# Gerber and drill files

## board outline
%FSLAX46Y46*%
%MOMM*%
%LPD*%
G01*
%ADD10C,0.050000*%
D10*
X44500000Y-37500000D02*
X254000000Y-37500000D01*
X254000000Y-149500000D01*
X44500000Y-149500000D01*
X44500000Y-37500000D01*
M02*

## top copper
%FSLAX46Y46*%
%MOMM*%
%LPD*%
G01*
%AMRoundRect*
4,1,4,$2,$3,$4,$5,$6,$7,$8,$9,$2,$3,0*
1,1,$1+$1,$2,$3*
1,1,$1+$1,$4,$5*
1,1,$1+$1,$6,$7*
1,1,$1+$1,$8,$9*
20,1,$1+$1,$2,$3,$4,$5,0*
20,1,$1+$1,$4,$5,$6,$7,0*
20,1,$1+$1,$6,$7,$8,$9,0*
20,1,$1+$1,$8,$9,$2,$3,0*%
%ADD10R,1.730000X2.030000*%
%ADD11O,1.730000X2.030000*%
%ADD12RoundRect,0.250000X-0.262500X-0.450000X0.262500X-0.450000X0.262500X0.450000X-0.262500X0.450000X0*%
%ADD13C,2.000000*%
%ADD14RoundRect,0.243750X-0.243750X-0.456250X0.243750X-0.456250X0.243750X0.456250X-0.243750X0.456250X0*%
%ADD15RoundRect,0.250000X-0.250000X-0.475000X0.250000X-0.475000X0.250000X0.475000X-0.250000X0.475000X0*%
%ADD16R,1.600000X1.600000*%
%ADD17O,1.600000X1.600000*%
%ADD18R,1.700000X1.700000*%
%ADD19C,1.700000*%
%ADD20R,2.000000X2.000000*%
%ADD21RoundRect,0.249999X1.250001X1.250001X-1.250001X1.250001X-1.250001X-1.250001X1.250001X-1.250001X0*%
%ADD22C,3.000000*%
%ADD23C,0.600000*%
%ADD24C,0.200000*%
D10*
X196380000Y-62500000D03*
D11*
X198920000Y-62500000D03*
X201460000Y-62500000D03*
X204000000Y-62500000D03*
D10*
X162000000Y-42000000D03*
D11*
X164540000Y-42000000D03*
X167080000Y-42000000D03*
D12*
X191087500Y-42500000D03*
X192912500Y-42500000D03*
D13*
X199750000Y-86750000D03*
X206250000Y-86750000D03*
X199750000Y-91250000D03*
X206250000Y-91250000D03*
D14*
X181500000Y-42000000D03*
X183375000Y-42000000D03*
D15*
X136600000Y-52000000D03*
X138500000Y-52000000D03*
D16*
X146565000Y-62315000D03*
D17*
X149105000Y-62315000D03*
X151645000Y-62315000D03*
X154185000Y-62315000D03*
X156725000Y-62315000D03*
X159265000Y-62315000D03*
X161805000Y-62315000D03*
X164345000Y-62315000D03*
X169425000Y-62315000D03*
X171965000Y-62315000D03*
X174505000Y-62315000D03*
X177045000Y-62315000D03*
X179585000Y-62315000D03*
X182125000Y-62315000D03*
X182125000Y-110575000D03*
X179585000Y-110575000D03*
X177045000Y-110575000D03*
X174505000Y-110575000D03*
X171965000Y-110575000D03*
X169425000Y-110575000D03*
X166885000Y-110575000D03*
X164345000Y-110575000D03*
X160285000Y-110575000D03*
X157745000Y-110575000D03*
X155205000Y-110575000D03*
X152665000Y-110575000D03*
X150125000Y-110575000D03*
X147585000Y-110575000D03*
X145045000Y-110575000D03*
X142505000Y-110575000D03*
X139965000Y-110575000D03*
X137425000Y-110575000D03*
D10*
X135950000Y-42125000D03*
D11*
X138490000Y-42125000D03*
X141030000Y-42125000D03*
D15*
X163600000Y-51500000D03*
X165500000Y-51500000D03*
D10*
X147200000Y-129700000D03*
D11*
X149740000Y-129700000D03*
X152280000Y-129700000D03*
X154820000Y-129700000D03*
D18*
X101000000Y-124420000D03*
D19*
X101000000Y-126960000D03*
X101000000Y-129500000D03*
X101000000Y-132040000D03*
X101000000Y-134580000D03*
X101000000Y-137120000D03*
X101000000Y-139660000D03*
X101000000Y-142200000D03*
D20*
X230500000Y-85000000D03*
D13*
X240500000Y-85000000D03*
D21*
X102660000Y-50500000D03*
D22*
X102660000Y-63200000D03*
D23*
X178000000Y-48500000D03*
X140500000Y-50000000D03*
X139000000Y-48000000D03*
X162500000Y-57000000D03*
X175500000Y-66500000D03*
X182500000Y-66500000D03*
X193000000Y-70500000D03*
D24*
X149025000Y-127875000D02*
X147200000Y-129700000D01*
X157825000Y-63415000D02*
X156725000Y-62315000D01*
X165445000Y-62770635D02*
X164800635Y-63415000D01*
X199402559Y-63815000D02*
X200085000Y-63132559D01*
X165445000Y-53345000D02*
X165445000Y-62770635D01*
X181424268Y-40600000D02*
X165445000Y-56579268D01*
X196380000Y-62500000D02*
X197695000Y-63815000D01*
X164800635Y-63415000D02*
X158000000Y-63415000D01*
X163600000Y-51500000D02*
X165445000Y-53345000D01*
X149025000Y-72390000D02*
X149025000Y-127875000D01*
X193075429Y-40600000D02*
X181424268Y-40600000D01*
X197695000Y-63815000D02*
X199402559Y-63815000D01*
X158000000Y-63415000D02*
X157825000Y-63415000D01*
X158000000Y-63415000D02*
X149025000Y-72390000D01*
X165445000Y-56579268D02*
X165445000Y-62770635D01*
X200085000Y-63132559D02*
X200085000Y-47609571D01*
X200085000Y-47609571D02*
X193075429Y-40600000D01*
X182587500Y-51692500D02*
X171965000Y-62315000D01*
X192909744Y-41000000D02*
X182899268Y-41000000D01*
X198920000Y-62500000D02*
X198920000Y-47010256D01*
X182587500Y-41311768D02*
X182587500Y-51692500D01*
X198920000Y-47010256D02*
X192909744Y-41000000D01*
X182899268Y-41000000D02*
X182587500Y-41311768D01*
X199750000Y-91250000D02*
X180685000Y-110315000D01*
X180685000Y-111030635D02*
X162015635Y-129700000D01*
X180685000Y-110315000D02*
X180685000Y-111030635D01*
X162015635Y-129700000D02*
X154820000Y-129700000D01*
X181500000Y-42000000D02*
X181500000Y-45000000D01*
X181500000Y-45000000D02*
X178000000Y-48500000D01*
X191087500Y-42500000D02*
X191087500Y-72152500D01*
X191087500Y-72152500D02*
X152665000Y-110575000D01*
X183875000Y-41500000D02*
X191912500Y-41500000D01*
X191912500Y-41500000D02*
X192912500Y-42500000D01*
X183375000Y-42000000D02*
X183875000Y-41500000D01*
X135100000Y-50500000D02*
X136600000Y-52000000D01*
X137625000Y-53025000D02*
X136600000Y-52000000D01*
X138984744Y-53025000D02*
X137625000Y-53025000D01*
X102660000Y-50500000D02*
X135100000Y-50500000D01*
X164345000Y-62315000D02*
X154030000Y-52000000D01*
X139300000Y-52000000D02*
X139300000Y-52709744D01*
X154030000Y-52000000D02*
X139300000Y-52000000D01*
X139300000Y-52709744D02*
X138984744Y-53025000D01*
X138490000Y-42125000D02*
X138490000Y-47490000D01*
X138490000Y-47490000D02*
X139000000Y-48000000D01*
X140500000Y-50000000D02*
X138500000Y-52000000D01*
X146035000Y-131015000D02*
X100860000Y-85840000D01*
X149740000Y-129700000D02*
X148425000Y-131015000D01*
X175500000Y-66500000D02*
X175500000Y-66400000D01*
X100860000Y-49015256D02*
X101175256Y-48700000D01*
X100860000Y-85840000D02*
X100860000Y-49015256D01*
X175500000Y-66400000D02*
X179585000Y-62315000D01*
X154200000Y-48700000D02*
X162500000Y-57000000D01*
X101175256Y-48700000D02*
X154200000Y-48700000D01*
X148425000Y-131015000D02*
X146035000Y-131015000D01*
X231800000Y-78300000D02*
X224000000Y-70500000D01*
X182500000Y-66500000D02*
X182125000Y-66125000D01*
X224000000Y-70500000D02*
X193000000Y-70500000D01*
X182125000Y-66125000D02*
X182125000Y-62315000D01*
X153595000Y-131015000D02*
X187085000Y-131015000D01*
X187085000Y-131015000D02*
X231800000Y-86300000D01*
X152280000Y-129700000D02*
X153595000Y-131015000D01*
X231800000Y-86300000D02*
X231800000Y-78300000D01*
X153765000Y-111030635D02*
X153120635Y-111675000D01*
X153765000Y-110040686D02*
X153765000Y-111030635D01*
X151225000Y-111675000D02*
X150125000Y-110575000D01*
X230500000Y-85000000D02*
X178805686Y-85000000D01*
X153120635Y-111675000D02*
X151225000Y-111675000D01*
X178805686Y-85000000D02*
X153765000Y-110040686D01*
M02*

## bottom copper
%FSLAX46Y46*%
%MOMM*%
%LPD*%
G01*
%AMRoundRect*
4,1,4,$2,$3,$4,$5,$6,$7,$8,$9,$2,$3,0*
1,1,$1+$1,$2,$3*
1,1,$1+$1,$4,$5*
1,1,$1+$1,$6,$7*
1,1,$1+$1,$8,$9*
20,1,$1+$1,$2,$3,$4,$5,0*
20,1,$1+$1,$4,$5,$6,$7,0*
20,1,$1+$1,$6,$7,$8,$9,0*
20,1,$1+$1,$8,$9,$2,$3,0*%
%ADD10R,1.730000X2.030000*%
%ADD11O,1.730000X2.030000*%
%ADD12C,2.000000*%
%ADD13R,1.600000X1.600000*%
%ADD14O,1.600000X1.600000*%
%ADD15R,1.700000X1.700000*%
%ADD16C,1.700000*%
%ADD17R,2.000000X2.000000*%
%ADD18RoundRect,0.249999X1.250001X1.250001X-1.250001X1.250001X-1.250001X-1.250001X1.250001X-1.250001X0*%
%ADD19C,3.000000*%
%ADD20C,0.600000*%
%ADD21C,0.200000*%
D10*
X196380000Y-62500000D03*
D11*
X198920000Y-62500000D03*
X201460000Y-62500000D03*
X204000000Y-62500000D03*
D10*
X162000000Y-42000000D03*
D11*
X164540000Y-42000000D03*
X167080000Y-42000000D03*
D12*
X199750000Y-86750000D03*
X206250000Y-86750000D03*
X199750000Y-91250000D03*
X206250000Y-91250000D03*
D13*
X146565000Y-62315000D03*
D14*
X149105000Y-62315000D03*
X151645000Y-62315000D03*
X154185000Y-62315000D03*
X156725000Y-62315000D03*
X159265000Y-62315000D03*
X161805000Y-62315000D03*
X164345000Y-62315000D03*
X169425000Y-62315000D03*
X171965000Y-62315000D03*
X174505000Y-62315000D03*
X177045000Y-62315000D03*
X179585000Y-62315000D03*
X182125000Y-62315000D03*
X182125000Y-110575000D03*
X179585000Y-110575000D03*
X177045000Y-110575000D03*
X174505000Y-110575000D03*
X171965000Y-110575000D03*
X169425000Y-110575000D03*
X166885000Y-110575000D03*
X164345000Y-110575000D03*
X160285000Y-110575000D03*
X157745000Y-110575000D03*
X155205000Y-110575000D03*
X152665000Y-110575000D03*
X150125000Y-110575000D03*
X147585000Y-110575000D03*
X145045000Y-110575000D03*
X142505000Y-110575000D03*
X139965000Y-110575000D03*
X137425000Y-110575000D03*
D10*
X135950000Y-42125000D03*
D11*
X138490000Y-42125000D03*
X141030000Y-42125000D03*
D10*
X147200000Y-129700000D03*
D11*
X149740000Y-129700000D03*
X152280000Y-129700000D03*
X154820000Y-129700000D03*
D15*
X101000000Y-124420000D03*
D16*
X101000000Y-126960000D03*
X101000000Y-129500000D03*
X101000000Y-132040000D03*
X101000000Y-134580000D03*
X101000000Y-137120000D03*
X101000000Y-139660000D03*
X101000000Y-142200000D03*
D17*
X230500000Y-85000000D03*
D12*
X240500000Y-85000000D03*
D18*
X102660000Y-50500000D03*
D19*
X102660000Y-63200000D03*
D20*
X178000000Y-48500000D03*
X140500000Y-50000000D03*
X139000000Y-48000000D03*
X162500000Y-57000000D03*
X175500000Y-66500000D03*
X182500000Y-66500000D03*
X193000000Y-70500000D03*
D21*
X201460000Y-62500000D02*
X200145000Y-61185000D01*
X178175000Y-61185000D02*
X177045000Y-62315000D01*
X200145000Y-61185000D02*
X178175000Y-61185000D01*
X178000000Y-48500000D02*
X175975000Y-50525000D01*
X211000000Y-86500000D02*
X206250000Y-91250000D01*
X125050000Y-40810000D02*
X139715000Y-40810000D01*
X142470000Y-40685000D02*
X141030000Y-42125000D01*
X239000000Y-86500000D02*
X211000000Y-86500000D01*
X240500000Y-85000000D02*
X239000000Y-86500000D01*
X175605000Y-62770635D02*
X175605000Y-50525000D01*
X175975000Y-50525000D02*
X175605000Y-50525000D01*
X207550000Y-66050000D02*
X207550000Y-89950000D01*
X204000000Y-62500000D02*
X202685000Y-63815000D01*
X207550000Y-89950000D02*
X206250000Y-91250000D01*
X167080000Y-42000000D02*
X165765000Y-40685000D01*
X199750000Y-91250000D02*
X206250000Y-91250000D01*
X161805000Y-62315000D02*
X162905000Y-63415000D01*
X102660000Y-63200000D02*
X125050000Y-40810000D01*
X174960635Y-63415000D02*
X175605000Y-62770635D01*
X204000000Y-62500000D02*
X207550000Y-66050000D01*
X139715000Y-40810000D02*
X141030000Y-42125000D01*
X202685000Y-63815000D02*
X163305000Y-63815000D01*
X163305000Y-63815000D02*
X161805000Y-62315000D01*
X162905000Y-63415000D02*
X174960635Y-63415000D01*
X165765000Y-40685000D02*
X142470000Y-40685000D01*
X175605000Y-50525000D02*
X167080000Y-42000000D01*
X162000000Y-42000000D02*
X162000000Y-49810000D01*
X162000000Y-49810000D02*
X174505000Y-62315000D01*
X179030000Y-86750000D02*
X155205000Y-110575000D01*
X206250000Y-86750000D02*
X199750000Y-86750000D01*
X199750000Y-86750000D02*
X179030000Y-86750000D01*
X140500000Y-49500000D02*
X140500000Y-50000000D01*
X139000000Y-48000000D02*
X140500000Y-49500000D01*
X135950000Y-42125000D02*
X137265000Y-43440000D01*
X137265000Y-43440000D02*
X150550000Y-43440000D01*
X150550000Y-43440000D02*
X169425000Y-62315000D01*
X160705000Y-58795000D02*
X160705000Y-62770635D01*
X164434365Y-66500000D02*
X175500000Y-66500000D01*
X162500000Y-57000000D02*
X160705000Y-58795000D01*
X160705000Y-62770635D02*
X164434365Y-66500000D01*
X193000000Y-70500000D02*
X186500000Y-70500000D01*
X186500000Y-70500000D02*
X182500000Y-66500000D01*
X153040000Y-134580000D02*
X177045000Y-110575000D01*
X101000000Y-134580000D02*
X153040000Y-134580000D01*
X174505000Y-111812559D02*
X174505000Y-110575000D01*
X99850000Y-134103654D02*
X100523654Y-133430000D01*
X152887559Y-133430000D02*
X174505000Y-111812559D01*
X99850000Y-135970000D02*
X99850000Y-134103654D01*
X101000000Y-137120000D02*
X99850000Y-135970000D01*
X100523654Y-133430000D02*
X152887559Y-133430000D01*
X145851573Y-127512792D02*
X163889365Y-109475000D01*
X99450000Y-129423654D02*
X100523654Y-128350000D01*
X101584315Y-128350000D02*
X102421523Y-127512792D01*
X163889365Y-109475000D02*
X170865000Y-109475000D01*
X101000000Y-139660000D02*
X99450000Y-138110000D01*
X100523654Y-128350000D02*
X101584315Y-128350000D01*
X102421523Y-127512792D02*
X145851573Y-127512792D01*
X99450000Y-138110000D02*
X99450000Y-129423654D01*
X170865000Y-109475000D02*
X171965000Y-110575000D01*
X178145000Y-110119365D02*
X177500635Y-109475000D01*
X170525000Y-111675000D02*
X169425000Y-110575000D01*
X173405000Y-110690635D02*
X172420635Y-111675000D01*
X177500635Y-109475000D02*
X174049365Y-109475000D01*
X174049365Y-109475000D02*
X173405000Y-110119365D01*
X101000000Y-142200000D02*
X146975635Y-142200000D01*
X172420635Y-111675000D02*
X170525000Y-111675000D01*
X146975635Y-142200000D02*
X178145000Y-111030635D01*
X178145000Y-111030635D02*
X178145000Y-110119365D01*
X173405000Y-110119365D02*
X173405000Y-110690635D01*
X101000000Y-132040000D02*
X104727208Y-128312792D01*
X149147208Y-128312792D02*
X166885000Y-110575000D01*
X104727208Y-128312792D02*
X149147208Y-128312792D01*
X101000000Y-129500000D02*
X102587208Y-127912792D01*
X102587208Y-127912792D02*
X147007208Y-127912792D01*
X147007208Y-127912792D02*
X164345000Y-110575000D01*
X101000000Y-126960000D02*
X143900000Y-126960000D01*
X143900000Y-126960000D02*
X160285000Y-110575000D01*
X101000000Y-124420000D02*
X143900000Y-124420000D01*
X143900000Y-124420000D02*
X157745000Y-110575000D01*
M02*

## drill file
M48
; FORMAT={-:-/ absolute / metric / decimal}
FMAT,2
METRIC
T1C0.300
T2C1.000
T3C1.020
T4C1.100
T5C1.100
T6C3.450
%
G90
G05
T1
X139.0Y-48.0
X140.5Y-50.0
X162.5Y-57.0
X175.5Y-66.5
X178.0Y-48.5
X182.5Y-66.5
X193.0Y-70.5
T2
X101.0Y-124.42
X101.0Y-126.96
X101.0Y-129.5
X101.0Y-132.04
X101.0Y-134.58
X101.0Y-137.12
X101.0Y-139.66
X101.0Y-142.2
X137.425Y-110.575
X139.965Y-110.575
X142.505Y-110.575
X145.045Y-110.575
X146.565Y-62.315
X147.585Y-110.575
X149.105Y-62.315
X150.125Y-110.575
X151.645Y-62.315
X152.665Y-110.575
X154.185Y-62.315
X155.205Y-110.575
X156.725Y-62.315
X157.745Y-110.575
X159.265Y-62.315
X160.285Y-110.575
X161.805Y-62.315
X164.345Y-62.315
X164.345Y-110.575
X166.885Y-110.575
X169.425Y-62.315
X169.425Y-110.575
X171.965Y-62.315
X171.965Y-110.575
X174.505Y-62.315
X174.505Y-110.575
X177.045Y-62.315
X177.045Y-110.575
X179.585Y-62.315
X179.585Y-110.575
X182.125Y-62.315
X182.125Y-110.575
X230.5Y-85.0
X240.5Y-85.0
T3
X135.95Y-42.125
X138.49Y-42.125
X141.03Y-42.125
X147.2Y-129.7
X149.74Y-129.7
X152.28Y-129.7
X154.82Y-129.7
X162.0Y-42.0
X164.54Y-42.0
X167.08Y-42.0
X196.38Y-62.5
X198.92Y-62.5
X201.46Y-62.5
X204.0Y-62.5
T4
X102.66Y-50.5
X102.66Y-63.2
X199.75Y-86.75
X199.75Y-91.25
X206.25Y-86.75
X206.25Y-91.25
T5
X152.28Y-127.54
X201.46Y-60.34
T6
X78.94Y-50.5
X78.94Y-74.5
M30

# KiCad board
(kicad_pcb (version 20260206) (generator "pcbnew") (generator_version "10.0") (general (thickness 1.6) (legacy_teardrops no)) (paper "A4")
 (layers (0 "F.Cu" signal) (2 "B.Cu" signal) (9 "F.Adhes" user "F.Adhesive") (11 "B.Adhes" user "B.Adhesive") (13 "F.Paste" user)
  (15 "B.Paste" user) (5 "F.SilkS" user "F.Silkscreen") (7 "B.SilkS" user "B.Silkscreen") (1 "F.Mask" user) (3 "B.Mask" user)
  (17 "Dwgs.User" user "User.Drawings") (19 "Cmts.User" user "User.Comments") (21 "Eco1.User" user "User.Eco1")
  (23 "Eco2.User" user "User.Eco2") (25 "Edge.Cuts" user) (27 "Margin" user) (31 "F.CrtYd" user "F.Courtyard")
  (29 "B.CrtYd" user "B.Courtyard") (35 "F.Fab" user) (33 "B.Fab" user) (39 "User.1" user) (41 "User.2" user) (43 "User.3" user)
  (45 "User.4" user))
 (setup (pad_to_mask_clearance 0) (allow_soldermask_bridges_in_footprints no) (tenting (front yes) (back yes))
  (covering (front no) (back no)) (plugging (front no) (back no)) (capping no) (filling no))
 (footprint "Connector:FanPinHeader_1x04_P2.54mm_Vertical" (layer "F.Cu") (at 196.38 62.5)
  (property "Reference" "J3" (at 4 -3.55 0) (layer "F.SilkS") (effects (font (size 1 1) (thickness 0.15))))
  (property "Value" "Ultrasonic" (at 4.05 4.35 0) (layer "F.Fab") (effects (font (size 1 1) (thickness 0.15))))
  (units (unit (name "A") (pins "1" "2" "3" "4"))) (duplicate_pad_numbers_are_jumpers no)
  (pad "" np_thru_hole circle (at 5.08 -2.16 90) (size 1.1 1.1) (drill 1.1) (layers "*.Cu" "*.Mask"))
  (pad "1" thru_hole rect (at 0 0 90) (size 2.03 1.73) (drill 1.02) (layers "*.Cu" "*.Mask") (remove_unused_layers no) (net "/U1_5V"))
  (pad "2" thru_hole oval (at 2.54 0 90) (size 2.03 1.73) (drill 1.02) (layers "*.Cu" "*.Mask") (remove_unused_layers no)
   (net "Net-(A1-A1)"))
  (pad "3" thru_hole oval (at 5.08 0 90) (size 2.03 1.73) (drill 1.02) (layers "*.Cu" "*.Mask") (remove_unused_layers no)
   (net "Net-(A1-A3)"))
  (pad "4" thru_hole oval (at 7.62 0 90) (size 2.03 1.73) (drill 1.02) (layers "*.Cu" "*.Mask") (remove_unused_layers no) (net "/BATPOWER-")))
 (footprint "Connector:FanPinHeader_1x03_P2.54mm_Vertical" (layer "F.Cu") (at 162 42)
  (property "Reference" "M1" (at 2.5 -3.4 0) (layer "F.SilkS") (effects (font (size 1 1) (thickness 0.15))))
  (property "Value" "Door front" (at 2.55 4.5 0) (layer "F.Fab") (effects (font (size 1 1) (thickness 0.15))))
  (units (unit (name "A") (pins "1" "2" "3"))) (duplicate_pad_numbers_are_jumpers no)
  (pad "1" thru_hole rect (at 0 0 90) (size 2.03 1.73) (drill 1.02) (layers "*.Cu" "*.Mask") (remove_unused_layers no) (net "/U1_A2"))
  (pad "2" thru_hole oval (at 2.54 0 90) (size 2.03 1.73) (drill 1.02) (layers "*.Cu" "*.Mask") (remove_unused_layers no) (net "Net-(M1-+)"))
  (pad "3" thru_hole oval (at 5.08 0 90) (size 2.03 1.73) (drill 1.02) (layers "*.Cu" "*.Mask") (remove_unused_layers no) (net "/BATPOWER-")))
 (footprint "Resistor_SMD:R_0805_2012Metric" (layer "F.Cu") (at 192 42.5)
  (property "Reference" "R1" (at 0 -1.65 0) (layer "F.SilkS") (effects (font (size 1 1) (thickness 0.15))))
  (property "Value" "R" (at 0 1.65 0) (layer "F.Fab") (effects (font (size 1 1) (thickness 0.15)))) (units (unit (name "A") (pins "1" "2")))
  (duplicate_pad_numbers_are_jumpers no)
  (pad "1" smd roundrect (at -0.9125 0) (size 1.025 1.4) (layers "F.Cu" "F.Mask" "F.Paste") (roundrect_rratio 0.243902) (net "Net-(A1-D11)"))
  (pad "2" smd roundrect (at 0.9125 0) (size 1.025 1.4) (layers "F.Cu" "F.Mask" "F.Paste") (roundrect_rratio 0.243902) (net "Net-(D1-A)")))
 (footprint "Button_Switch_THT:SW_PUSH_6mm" (layer "F.Cu") (at 199.75 86.75)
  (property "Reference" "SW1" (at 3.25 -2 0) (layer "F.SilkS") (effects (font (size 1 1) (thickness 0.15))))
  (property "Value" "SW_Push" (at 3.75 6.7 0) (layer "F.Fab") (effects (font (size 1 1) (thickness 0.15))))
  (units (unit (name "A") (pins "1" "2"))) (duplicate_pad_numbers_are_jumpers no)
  (pad "1" thru_hole circle (at 0 0 90) (size 2 2) (drill 1.1) (layers "*.Cu" "*.Mask") (remove_unused_layers no) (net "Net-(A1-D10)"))
  (pad "1" thru_hole circle (at 6.5 0 90) (size 2 2) (drill 1.1) (layers "*.Cu" "*.Mask") (remove_unused_layers no) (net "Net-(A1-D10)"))
  (pad "2" thru_hole circle (at 0 4.5 90) (size 2 2) (drill 1.1) (layers "*.Cu" "*.Mask") (remove_unused_layers no) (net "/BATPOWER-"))
  (pad "2" thru_hole circle (at 6.5 4.5 90) (size 2 2) (drill 1.1) (layers "*.Cu" "*.Mask") (remove_unused_layers no) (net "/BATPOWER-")))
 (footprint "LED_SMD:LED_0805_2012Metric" (layer "F.Cu") (at 182.4375 42)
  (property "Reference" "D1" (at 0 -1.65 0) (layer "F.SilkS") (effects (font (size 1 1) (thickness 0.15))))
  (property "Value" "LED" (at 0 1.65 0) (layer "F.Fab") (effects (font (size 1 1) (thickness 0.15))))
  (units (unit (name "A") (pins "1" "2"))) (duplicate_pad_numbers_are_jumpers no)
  (pad "1" smd roundrect (at -0.9375 0) (size 0.975 1.4) (layers "F.Cu" "F.Mask" "F.Paste") (roundrect_rratio 0.25) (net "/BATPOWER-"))
  (pad "2" smd roundrect (at 0.9375 0) (size 0.975 1.4) (layers "F.Cu" "F.Mask" "F.Paste") (roundrect_rratio 0.25) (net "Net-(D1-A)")))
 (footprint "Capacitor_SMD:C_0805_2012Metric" (layer "F.Cu") (at 137.55 52)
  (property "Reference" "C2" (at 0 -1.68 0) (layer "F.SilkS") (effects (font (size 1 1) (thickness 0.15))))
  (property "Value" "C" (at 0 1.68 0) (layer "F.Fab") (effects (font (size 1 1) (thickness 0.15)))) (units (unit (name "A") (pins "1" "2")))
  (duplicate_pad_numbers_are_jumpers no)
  (pad "1" smd roundrect (at -0.95 0) (size 1 1.45) (layers "F.Cu" "F.Mask" "F.Paste") (roundrect_rratio 0.25) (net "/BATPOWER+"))
  (pad "2" smd roundrect (at 0.95 0) (size 1 1.45) (layers "F.Cu" "F.Mask" "F.Paste") (roundrect_rratio 0.25) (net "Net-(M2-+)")))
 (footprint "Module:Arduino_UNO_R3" (layer "F.Cu") (at 146.565 62.315)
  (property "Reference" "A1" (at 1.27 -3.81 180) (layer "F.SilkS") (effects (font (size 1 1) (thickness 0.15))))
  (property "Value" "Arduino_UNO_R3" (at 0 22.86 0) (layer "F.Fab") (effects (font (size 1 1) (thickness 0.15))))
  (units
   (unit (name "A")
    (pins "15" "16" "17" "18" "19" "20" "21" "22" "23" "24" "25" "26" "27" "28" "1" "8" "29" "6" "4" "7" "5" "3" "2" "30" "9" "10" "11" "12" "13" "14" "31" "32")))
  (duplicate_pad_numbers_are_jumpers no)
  (pad "1" thru_hole rect (at 0 0 90) (size 1.6 1.6) (drill 1) (layers "*.Cu" "*.Mask") (remove_unused_layers no)
   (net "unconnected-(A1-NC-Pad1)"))
  (pad "2" thru_hole oval (at 2.54 0 90) (size 1.6 1.6) (drill 1) (layers "*.Cu" "*.Mask") (remove_unused_layers no)
   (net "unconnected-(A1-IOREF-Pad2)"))
  (pad "3" thru_hole oval (at 5.08 0 90) (size 1.6 1.6) (drill 1) (layers "*.Cu" "*.Mask") (remove_unused_layers no)
   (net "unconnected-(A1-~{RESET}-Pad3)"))
  (pad "4" thru_hole oval (at 7.62 0 90) (size 1.6 1.6) (drill 1) (layers "*.Cu" "*.Mask") (remove_unused_layers no)
   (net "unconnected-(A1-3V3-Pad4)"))
  (pad "5" thru_hole oval (at 10.16 0 90) (size 1.6 1.6) (drill 1) (layers "*.Cu" "*.Mask") (remove_unused_layers no) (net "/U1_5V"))
  (pad "6" thru_hole oval (at 12.7 0 90) (size 1.6 1.6) (drill 1) (layers "*.Cu" "*.Mask") (remove_unused_layers no)
   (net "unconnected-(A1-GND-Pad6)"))
  (pad "7" thru_hole oval (at 15.24 0 90) (size 1.6 1.6) (drill 1) (layers "*.Cu" "*.Mask") (remove_unused_layers no) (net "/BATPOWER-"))
  (pad "8" thru_hole oval (at 17.78 0 90) (size 1.6 1.6) (drill 1) (layers "*.Cu" "*.Mask") (remove_unused_layers no) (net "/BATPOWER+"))
  (pad "9" thru_hole oval (at 22.86 0 90) (size 1.6 1.6) (drill 1) (layers "*.Cu" "*.Mask") (remove_unused_layers no) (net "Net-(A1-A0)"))
  (pad "10" thru_hole oval (at 25.4 0 90) (size 1.6 1.6) (drill 1) (layers "*.Cu" "*.Mask") (remove_unused_layers no) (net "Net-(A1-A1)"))
  (pad "11" thru_hole oval (at 27.94 0 90) (size 1.6 1.6) (drill 1) (layers "*.Cu" "*.Mask") (remove_unused_layers no) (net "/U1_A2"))
  (pad "12" thru_hole oval (at 30.48 0 90) (size 1.6 1.6) (drill 1) (layers "*.Cu" "*.Mask") (remove_unused_layers no) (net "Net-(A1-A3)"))
  (pad "13" thru_hole oval (at 33.02 0 90) (size 1.6 1.6) (drill 1) (layers "*.Cu" "*.Mask") (remove_unused_layers no) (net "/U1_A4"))
  (pad "14" thru_hole oval (at 35.56 0 90) (size 1.6 1.6) (drill 1) (layers "*.Cu" "*.Mask") (remove_unused_layers no) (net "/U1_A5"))
  (pad "15" thru_hole oval (at 35.56 48.26 90) (size 1.6 1.6) (drill 1) (layers "*.Cu" "*.Mask") (remove_unused_layers no)
   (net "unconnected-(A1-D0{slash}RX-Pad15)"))
  (pad "16" thru_hole oval (at 33.02 48.26 90) (size 1.6 1.6) (drill 1) (layers "*.Cu" "*.Mask") (remove_unused_layers no)
   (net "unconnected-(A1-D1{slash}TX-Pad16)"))
  (pad "17" thru_hole oval (at 30.48 48.26 90) (size 1.6 1.6) (drill 1) (layers "*.Cu" "*.Mask") (remove_unused_layers no) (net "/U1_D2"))
  (pad "18" thru_hole oval (at 27.94 48.26 90) (size 1.6 1.6) (drill 1) (layers "*.Cu" "*.Mask") (remove_unused_layers no) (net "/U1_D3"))
  (pad "19" thru_hole oval (at 25.4 48.26 90) (size 1.6 1.6) (drill 1) (layers "*.Cu" "*.Mask") (remove_unused_layers no) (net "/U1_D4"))
  (pad "20" thru_hole oval (at 22.86 48.26 90) (size 1.6 1.6) (drill 1) (layers "*.Cu" "*.Mask") (remove_unused_layers no) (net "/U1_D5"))
  (pad "21" thru_hole oval (at 20.32 48.26 90) (size 1.6 1.6) (drill 1) (layers "*.Cu" "*.Mask") (remove_unused_layers no) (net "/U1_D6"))
  (pad "22" thru_hole oval (at 17.78 48.26 90) (size 1.6 1.6) (drill 1) (layers "*.Cu" "*.Mask") (remove_unused_layers no) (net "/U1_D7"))
  (pad "23" thru_hole oval (at 13.72 48.26 90) (size 1.6 1.6) (drill 1) (layers "*.Cu" "*.Mask") (remove_unused_layers no) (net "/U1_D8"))
  (pad "24" thru_hole oval (at 11.18 48.26 90) (size 1.6 1.6) (drill 1) (layers "*.Cu" "*.Mask") (remove_unused_layers no) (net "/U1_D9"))
  (pad "25" thru_hole oval (at 8.64 48.26 90) (size 1.6 1.6) (drill 1) (layers "*.Cu" "*.Mask") (remove_unused_layers no)
   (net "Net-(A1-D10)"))
  (pad "26" thru_hole oval (at 6.1 48.26 90) (size 1.6 1.6) (drill 1) (layers "*.Cu" "*.Mask") (remove_unused_layers no)
   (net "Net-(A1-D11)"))
  (pad "27" thru_hole oval (at 3.56 48.26 90) (size 1.6 1.6) (drill 1) (layers "*.Cu" "*.Mask") (remove_unused_layers no) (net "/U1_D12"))
  (pad "28" thru_hole oval (at 1.02 48.26 90) (size 1.6 1.6) (drill 1) (layers "*.Cu" "*.Mask") (remove_unused_layers no)
   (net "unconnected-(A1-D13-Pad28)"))
  (pad "29" thru_hole oval (at -1.52 48.26 90) (size 1.6 1.6) (drill 1) (layers "*.Cu" "*.Mask") (remove_unused_layers no)
   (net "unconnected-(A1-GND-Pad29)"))
  (pad "30" thru_hole oval (at -4.06 48.26 90) (size 1.6 1.6) (drill 1) (layers "*.Cu" "*.Mask") (remove_unused_layers no)
   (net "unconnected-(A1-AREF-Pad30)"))
  (pad "31" thru_hole oval (at -6.6 48.26 90) (size 1.6 1.6) (drill 1) (layers "*.Cu" "*.Mask") (remove_unused_layers no)
   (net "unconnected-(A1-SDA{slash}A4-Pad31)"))
  (pad "32" thru_hole oval (at -9.14 48.26 90) (size 1.6 1.6) (drill 1) (layers "*.Cu" "*.Mask") (remove_unused_layers no)
   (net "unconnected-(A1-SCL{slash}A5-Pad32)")))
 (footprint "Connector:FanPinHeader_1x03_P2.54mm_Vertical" (layer "F.Cu") (at 135.95 42.125)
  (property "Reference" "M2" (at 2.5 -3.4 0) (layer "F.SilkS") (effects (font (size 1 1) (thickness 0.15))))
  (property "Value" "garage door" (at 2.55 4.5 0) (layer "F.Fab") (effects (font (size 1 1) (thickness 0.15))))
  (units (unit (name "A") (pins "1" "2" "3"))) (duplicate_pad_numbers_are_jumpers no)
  (pad "1" thru_hole rect (at 0 0 90) (size 2.03 1.73) (drill 1.02) (layers "*.Cu" "*.Mask") (remove_unused_layers no) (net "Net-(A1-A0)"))
  (pad "2" thru_hole oval (at 2.54 0 90) (size 2.03 1.73) (drill 1.02) (layers "*.Cu" "*.Mask") (remove_unused_layers no) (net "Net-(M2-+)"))
  (pad "3" thru_hole oval (at 5.08 0 90) (size 2.03 1.73) (drill 1.02) (layers "*.Cu" "*.Mask") (remove_unused_layers no) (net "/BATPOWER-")))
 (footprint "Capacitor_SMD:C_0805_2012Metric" (layer "F.Cu") (at 164.55 51.5)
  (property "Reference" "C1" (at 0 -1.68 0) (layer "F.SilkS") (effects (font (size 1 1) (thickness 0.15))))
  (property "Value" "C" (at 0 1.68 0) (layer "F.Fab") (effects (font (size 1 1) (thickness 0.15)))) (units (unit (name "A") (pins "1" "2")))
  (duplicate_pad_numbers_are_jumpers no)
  (pad "1" smd roundrect (at -0.95 0) (size 1 1.45) (layers "F.Cu" "F.Mask" "F.Paste") (roundrect_rratio 0.25) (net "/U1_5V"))
  (pad "2" smd roundrect (at 0.95 0) (size 1 1.45) (layers "F.Cu" "F.Mask" "F.Paste") (roundrect_rratio 0.25) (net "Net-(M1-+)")))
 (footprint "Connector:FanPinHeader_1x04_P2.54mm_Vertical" (layer "F.Cu") (at 147.2 129.7)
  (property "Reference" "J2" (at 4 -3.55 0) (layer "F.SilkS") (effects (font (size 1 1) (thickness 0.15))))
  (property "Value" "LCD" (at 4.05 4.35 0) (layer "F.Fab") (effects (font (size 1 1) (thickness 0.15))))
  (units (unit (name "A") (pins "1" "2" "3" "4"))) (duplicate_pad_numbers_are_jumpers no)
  (pad "" np_thru_hole circle (at 5.08 -2.16 90) (size 1.1 1.1) (drill 1.1) (layers "*.Cu" "*.Mask"))
  (pad "1" thru_hole rect (at 0 0 90) (size 2.03 1.73) (drill 1.02) (layers "*.Cu" "*.Mask") (remove_unused_layers no) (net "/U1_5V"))
  (pad "2" thru_hole oval (at 2.54 0 90) (size 2.03 1.73) (drill 1.02) (layers "*.Cu" "*.Mask") (remove_unused_layers no) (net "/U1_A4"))
  (pad "3" thru_hole oval (at 5.08 0 90) (size 2.03 1.73) (drill 1.02) (layers "*.Cu" "*.Mask") (remove_unused_layers no) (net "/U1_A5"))
  (pad "4" thru_hole oval (at 7.62 0 90) (size 2.03 1.73) (drill 1.02) (layers "*.Cu" "*.Mask") (remove_unused_layers no) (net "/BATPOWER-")))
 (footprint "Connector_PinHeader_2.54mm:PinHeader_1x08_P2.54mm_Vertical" (layer "F.Cu") (at 101 124.42)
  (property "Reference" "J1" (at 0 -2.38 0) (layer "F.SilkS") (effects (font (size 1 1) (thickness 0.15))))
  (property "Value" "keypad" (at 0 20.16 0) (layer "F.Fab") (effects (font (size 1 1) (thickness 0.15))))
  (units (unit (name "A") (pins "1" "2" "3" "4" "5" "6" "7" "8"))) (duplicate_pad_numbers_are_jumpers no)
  (pad "1" thru_hole rect (at 0 0) (size 1.7 1.7) (drill 1) (layers "*.Cu" "*.Mask") (remove_unused_layers no) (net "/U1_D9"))
  (pad "2" thru_hole circle (at 0 2.54) (size 1.7 1.7) (drill 1) (layers "*.Cu" "*.Mask") (remove_unused_layers no) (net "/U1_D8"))
  (pad "3" thru_hole circle (at 0 5.08) (size 1.7 1.7) (drill 1) (layers "*.Cu" "*.Mask") (remove_unused_layers no) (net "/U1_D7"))
  (pad "4" thru_hole circle (at 0 7.62) (size 1.7 1.7) (drill 1) (layers "*.Cu" "*.Mask") (remove_unused_layers no) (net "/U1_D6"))
  (pad "5" thru_hole circle (at 0 10.16) (size 1.7 1.7) (drill 1) (layers "*.Cu" "*.Mask") (remove_unused_layers no) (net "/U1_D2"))
  (pad "6" thru_hole circle (at 0 12.7) (size 1.7 1.7) (drill 1) (layers "*.Cu" "*.Mask") (remove_unused_layers no) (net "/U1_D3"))
  (pad "7" thru_hole circle (at 0 15.24) (size 1.7 1.7) (drill 1) (layers "*.Cu" "*.Mask") (remove_unused_layers no) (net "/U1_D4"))
  (pad "8" thru_hole circle (at 0 17.78) (size 1.7 1.7) (drill 1) (layers "*.Cu" "*.Mask") (remove_unused_layers no) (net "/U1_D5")))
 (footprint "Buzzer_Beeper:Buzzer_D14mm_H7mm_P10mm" (layer "F.Cu") (at 230.5 85)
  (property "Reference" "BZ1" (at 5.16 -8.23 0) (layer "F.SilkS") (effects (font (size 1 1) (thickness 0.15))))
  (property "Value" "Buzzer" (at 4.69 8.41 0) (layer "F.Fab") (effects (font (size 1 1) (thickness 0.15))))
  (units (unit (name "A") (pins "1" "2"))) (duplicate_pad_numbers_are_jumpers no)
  (pad "1" thru_hole rect (at 0 0) (size 2 2) (drill 1) (layers "*.Cu" "*.Mask") (remove_unused_layers no) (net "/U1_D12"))
  (pad "2" thru_hole circle (at 10 0) (size 2 2) (drill 1) (layers "*.Cu" "*.Mask") (remove_unused_layers no) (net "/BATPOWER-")))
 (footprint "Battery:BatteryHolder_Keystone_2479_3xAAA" (layer "B.Cu") (at 102.66 50.5 180)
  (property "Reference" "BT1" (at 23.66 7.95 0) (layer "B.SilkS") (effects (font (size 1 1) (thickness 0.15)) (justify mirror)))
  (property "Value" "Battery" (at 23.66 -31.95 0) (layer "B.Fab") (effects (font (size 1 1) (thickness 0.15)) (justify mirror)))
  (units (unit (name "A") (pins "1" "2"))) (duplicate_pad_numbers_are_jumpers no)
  (pad "" np_thru_hole circle (at 23.72 -24 180) (size 3.45 3.45) (drill 3.45) (layers "*.Cu" "*.Mask"))
  (pad "" np_thru_hole circle (at 23.72 0 180) (size 3.45 3.45) (drill 3.45) (layers "*.Cu" "*.Mask"))
  (pad "1" thru_hole roundrect (at 0 0 180) (size 3 3) (drill 1.1) (layers "*.Cu" "*.Mask") (remove_unused_layers no)
   (roundrect_rratio 0.083333) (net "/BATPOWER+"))
  (pad "2" thru_hole circle (at 0 -12.7 180) (size 3 3) (drill 1.1) (layers "*.Cu" "*.Mask") (remove_unused_layers no) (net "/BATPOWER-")))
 (gr_rect (start 44.5 37.5) (end 254 149.5) (stroke (width 0.05) (type default)) (fill no) (layer "Edge.Cuts"))
 (segment (start 149.025 127.875) (end 147.2 129.7) (width 0.2) (layer "F.Cu") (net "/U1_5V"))
 (segment (start 157.825 63.415) (end 156.725 62.315) (width 0.2) (layer "F.Cu") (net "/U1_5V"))
 (segment (start 165.445 62.770635) (end 164.800635 63.415) (width 0.2) (layer "F.Cu") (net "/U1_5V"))
 (segment (start 199.402559 63.815) (end 200.085 63.132559) (width 0.2) (layer "F.Cu") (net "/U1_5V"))
 (segment (start 165.445 53.345) (end 165.445 62.770635) (width 0.2) (layer "F.Cu") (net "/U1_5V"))
 (segment (start 181.424268 40.6) (end 165.445 56.579268) (width 0.2) (layer "F.Cu") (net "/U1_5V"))
 (segment (start 196.38 62.5) (end 197.695 63.815) (width 0.2) (layer "F.Cu") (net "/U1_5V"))
 (segment (start 164.800635 63.415) (end 158 63.415) (width 0.2) (layer "F.Cu") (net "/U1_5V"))
 (segment (start 163.6 51.5) (end 165.445 53.345) (width 0.2) (layer "F.Cu") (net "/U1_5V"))
 (segment (start 149.025 72.39) (end 149.025 127.875) (width 0.2) (layer "F.Cu") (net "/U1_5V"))
 (segment (start 193.075429 40.6) (end 181.424268 40.6) (width 0.2) (layer "F.Cu") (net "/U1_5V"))
 (segment (start 197.695 63.815) (end 199.402559 63.815) (width 0.2) (layer "F.Cu") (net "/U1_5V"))
 (segment (start 158 63.415) (end 157.825 63.415) (width 0.2) (layer "F.Cu") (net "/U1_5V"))
 (segment (start 158 63.415) (end 149.025 72.39) (width 0.2) (layer "F.Cu") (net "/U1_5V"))
 (segment (start 165.445 56.579268) (end 165.445 62.770635) (width 0.2) (layer "F.Cu") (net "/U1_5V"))
 (segment (start 200.085 63.132559) (end 200.085 47.609571) (width 0.2) (layer "F.Cu") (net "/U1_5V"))
 (segment (start 200.085 47.609571) (end 193.075429 40.6) (width 0.2) (layer "F.Cu") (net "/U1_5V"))
 (segment (start 182.5875 51.6925) (end 171.965 62.315) (width 0.2) (layer "F.Cu") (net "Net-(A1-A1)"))
 (segment (start 192.909744 41) (end 182.899268 41) (width 0.2) (layer "F.Cu") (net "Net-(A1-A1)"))
 (segment (start 198.92 62.5) (end 198.92 47.010256) (width 0.2) (layer "F.Cu") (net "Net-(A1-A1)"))
 (segment (start 182.5875 41.311768) (end 182.5875 51.6925) (width 0.2) (layer "F.Cu") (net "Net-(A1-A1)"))
 (segment (start 198.92 47.010256) (end 192.909744 41) (width 0.2) (layer "F.Cu") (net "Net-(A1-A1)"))
 (segment (start 182.899268 41) (end 182.5875 41.311768) (width 0.2) (layer "F.Cu") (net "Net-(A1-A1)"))
 (segment (start 201.46 62.5) (end 200.145 61.185) (width 0.2) (layer "B.Cu") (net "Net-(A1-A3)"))
 (segment (start 178.175 61.185) (end 177.045 62.315) (width 0.2) (layer "B.Cu") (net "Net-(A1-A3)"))
 (segment (start 200.145 61.185) (end 178.175 61.185) (width 0.2) (layer "B.Cu") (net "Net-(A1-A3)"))
 (segment (start 199.75 91.25) (end 180.685 110.315) (width 0.2) (layer "F.Cu") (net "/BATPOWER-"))
 (segment (start 180.685 111.030635) (end 162.015635 129.7) (width 0.2) (layer "F.Cu") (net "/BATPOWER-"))
 (segment (start 180.685 110.315) (end 180.685 111.030635) (width 0.2) (layer "F.Cu") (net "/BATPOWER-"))
 (segment (start 162.015635 129.7) (end 154.82 129.7) (width 0.2) (layer "F.Cu") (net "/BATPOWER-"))
 (segment (start 181.5 42) (end 181.5 45) (width 0.2) (layer "F.Cu") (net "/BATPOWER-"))
 (segment (start 181.5 45) (end 178 48.5) (width 0.2) (layer "F.Cu") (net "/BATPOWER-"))
 (via (at 178 48.5) (size 0.6) (drill 0.3) (layers "F.Cu" "B.Cu") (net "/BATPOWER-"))
 (segment (start 178 48.5) (end 175.975 50.525) (width 0.2) (layer "B.Cu") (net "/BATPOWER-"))
 (segment (start 211 86.5) (end 206.25 91.25) (width 0.2) (layer "B.Cu") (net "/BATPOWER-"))
 (segment (start 125.05 40.81) (end 139.715 40.81) (width 0.2) (layer "B.Cu") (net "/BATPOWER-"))
 (segment (start 142.47 40.685) (end 141.03 42.125) (width 0.2) (layer "B.Cu") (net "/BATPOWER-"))
 (segment (start 239 86.5) (end 211 86.5) (width 0.2) (layer "B.Cu") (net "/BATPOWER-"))
 (segment (start 240.5 85) (end 239 86.5) (width 0.2) (layer "B.Cu") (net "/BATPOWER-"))
 (segment (start 175.605 62.770635) (end 175.605 50.525) (width 0.2) (layer "B.Cu") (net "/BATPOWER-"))
 (segment (start 175.975 50.525) (end 175.605 50.525) (width 0.2) (layer "B.Cu") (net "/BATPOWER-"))
 (segment (start 207.55 66.05) (end 207.55 89.95) (width 0.2) (layer "B.Cu") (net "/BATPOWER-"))
 (segment (start 204 62.5) (end 202.685 63.815) (width 0.2) (layer "B.Cu") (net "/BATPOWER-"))
 (segment (start 207.55 89.95) (end 206.25 91.25) (width 0.2) (layer "B.Cu") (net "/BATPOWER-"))
 (segment (start 167.08 42) (end 165.765 40.685) (width 0.2) (layer "B.Cu") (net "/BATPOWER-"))
 (segment (start 199.75 91.25) (end 206.25 91.25) (width 0.2) (layer "B.Cu") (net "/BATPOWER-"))
 (segment (start 161.805 62.315) (end 162.905 63.415) (width 0.2) (layer "B.Cu") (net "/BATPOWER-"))
 (segment (start 102.66 63.2) (end 125.05 40.81) (width 0.2) (layer "B.Cu") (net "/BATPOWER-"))
 (segment (start 174.960635 63.415) (end 175.605 62.770635) (width 0.2) (layer "B.Cu") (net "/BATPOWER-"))
 (segment (start 204 62.5) (end 207.55 66.05) (width 0.2) (layer "B.Cu") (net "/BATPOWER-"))
 (segment (start 139.715 40.81) (end 141.03 42.125) (width 0.2) (layer "B.Cu") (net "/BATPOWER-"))
 (segment (start 202.685 63.815) (end 163.305 63.815) (width 0.2) (layer "B.Cu") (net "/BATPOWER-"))
 (segment (start 163.305 63.815) (end 161.805 62.315) (width 0.2) (layer "B.Cu") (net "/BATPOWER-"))
 (segment (start 162.905 63.415) (end 174.960635 63.415) (width 0.2) (layer "B.Cu") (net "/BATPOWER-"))
 (segment (start 165.765 40.685) (end 142.47 40.685) (width 0.2) (layer "B.Cu") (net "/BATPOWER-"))
 (segment (start 175.605 50.525) (end 167.08 42) (width 0.2) (layer "B.Cu") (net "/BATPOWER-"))
 (segment (start 162 42) (end 162 49.81) (width 0.2) (layer "B.Cu") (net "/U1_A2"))
 (segment (start 162 49.81) (end 174.505 62.315) (width 0.2) (layer "B.Cu") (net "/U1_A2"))
 (segment (start 191.0875 42.5) (end 191.0875 72.1525) (width 0.2) (layer "F.Cu") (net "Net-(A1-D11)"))
 (segment (start 191.0875 72.1525) (end 152.665 110.575) (width 0.2) (layer "F.Cu") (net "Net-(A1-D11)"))
 (segment (start 183.875 41.5) (end 191.9125 41.5) (width 0.2) (layer "F.Cu") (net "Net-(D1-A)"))
 (segment (start 191.9125 41.5) (end 192.9125 42.5) (width 0.2) (layer "F.Cu") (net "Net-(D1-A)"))
 (segment (start 183.375 42) (end 183.875 41.5) (width 0.2) (layer "F.Cu") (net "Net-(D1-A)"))
 (segment (start 179.03 86.75) (end 155.205 110.575) (width 0.2) (layer "B.Cu") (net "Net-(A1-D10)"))
 (segment (start 206.25 86.75) (end 199.75 86.75) (width 0.2) (layer "B.Cu") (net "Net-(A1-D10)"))
 (segment (start 199.75 86.75) (end 179.03 86.75) (width 0.2) (layer "B.Cu") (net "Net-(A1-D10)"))
 (segment (start 135.1 50.5) (end 136.6 52) (width 0.2) (layer "F.Cu") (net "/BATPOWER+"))
 (segment (start 137.625 53.025) (end 136.6 52) (width 0.2) (layer "F.Cu") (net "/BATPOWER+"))
 (segment (start 138.984744 53.025) (end 137.625 53.025) (width 0.2) (layer "F.Cu") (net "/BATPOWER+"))
 (segment (start 102.66 50.5) (end 135.1 50.5) (width 0.2) (layer "F.Cu") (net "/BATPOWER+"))
 (segment (start 164.345 62.315) (end 154.03 52) (width 0.2) (layer "F.Cu") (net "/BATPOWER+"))
 (segment (start 139.3 52) (end 139.3 52.709744) (width 0.2) (layer "F.Cu") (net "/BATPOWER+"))
 (segment (start 154.03 52) (end 139.3 52) (width 0.2) (layer "F.Cu") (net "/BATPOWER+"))
 (segment (start 139.3 52.709744) (end 138.984744 53.025) (width 0.2) (layer "F.Cu") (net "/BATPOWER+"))
 (segment (start 138.49 42.125) (end 138.49 47.49) (width 0.2) (layer "F.Cu") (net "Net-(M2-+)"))
 (segment (start 138.49 47.49) (end 139 48) (width 0.2) (layer "F.Cu") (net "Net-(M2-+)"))
 (segment (start 140.5 50) (end 138.5 52) (width 0.2) (layer "F.Cu") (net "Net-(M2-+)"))
 (via (at 140.5 50) (size 0.6) (drill 0.3) (layers "F.Cu" "B.Cu") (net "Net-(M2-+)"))
 (via (at 139 48) (size 0.6) (drill 0.3) (layers "F.Cu" "B.Cu") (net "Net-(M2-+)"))
 (segment (start 140.5 49.5) (end 140.5 50) (width 0.2) (layer "B.Cu") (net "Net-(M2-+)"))
 (segment (start 139 48) (end 140.5 49.5) (width 0.2) (layer "B.Cu") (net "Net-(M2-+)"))
 (segment (start 135.95 42.125) (end 137.265 43.44) (width 0.2) (layer "B.Cu") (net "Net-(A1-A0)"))
 (segment (start 137.265 43.44) (end 150.55 43.44) (width 0.2) (layer "B.Cu") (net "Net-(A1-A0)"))
 (segment (start 150.55 43.44) (end 169.425 62.315) (width 0.2) (layer "B.Cu") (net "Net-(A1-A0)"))
 (segment (start 146.035 131.015) (end 100.86 85.84) (width 0.2) (layer "F.Cu") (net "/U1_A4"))
 (segment (start 149.74 129.7) (end 148.425 131.015) (width 0.2) (layer "F.Cu") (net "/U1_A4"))
 (segment (start 175.5 66.5) (end 175.5 66.4) (width 0.2) (layer "F.Cu") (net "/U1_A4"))
 (segment (start 100.86 49.015256) (end 101.175256 48.7) (width 0.2) (layer "F.Cu") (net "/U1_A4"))
 (segment (start 100.86 85.84) (end 100.86 49.015256) (width 0.2) (layer "F.Cu") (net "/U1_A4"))
 (segment (start 175.5 66.4) (end 179.585 62.315) (width 0.2) (layer "F.Cu") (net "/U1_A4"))
 (segment (start 154.2 48.7) (end 162.5 57) (width 0.2) (layer "F.Cu") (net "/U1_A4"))
 (segment (start 101.175256 48.7) (end 154.2 48.7) (width 0.2) (layer "F.Cu") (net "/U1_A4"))
 (segment (start 148.425 131.015) (end 146.035 131.015) (width 0.2) (layer "F.Cu") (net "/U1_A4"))
 (via (at 162.5 57) (size 0.6) (drill 0.3) (layers "F.Cu" "B.Cu") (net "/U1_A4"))
 (via (at 175.5 66.5) (size 0.6) (drill 0.3) (layers "F.Cu" "B.Cu") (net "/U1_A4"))
 (segment (start 160.705 58.795) (end 160.705 62.770635) (width 0.2) (layer "B.Cu") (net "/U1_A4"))
 (segment (start 164.434365 66.5) (end 175.5 66.5) (width 0.2) (layer "B.Cu") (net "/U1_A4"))
 (segment (start 162.5 57) (end 160.705 58.795) (width 0.2) (layer "B.Cu") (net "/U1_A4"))
 (segment (start 160.705 62.770635) (end 164.434365 66.5) (width 0.2) (layer "B.Cu") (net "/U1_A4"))
 (segment (start 231.8 78.3) (end 224 70.5) (width 0.2) (layer "F.Cu") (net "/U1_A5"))
 (segment (start 182.5 66.5) (end 182.125 66.125) (width 0.2) (layer "F.Cu") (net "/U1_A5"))
 (segment (start 224 70.5) (end 193 70.5) (width 0.2) (layer "F.Cu") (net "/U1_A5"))
 (segment (start 182.125 66.125) (end 182.125 62.315) (width 0.2) (layer "F.Cu") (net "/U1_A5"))
 (segment (start 153.595 131.015) (end 187.085 131.015) (width 0.2) (layer "F.Cu") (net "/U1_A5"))
 (segment (start 187.085 131.015) (end 231.8 86.3) (width 0.2) (layer "F.Cu") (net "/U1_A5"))
 (segment (start 152.28 129.7) (end 153.595 131.015) (width 0.2) (layer "F.Cu") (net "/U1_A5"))
 (segment (start 231.8 86.3) (end 231.8 78.3) (width 0.2) (layer "F.Cu") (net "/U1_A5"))
 (via (at 182.5 66.5) (size 0.6) (drill 0.3) (layers "F.Cu" "B.Cu") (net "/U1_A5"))
 (via (at 193 70.5) (size 0.6) (drill 0.3) (layers "F.Cu" "B.Cu") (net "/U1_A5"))
 (segment (start 193 70.5) (end 186.5 70.5) (width 0.2) (layer "B.Cu") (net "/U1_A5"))
 (segment (start 186.5 70.5) (end 182.5 66.5) (width 0.2) (layer "B.Cu") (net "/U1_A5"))
 (segment (start 153.04 134.58) (end 177.045 110.575) (width 0.2) (layer "B.Cu") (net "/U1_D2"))
 (segment (start 101 134.58) (end 153.04 134.58) (width 0.2) (layer "B.Cu") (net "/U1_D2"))
 (segment (start 174.505 111.812559) (end 174.505 110.575) (width 0.2) (layer "B.Cu") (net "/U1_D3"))
 (segment (start 99.85 134.103654) (end 100.523654 133.43) (width 0.2) (layer "B.Cu") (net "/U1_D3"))
 (segment (start 152.887559 133.43) (end 174.505 111.812559) (width 0.2) (layer "B.Cu") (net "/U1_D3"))
 (segment (start 99.85 135.97) (end 99.85 134.103654) (width 0.2) (layer "B.Cu") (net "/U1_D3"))
 (segment (start 101 137.12) (end 99.85 135.97) (width 0.2) (layer "B.Cu") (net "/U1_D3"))
 (segment (start 100.523654 133.43) (end 152.887559 133.43) (width 0.2) (layer "B.Cu") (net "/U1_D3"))
 (segment (start 145.851573 127.512792) (end 163.889365 109.475) (width 0.2) (layer "B.Cu") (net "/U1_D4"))
 (segment (start 99.45 129.423654) (end 100.523654 128.35) (width 0.2) (layer "B.Cu") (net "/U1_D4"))
 (segment (start 101.584315 128.35) (end 102.421523 127.512792) (width 0.2) (layer "B.Cu") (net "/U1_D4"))
 (segment (start 163.889365 109.475) (end 170.865 109.475) (width 0.2) (layer "B.Cu") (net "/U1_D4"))
 (segment (start 101 139.66) (end 99.45 138.11) (width 0.2) (layer "B.Cu") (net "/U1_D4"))
 (segment (start 100.523654 128.35) (end 101.584315 128.35) (width 0.2) (layer "B.Cu") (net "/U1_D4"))
 (segment (start 102.421523 127.512792) (end 145.851573 127.512792) (width 0.2) (layer "B.Cu") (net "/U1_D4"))
 (segment (start 99.45 138.11) (end 99.45 129.423654) (width 0.2) (layer "B.Cu") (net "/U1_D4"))
 (segment (start 170.865 109.475) (end 171.965 110.575) (width 0.2) (layer "B.Cu") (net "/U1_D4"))
 (segment (start 178.145 110.119365) (end 177.500635 109.475) (width 0.2) (layer "B.Cu") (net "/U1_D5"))
 (segment (start 170.525 111.675) (end 169.425 110.575) (width 0.2) (layer "B.Cu") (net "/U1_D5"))
 (segment (start 173.405 110.690635) (end 172.420635 111.675) (width 0.2) (layer "B.Cu") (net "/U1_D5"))
 (segment (start 177.500635 109.475) (end 174.049365 109.475) (width 0.2) (layer "B.Cu") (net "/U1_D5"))
 (segment (start 174.049365 109.475) (end 173.405 110.119365) (width 0.2) (layer "B.Cu") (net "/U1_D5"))
 (segment (start 101 142.2) (end 146.975635 142.2) (width 0.2) (layer "B.Cu") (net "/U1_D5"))
 (segment (start 172.420635 111.675) (end 170.525 111.675) (width 0.2) (layer "B.Cu") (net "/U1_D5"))
 (segment (start 146.975635 142.2) (end 178.145 111.030635) (width 0.2) (layer "B.Cu") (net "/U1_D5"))
 (segment (start 178.145 111.030635) (end 178.145 110.119365) (width 0.2) (layer "B.Cu") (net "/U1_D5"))
 (segment (start 173.405 110.119365) (end 173.405 110.690635) (width 0.2) (layer "B.Cu") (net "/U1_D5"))
 (segment (start 101 132.04) (end 104.727208 128.312792) (width 0.2) (layer "B.Cu") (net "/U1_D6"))
 (segment (start 149.147208 128.312792) (end 166.885 110.575) (width 0.2) (layer "B.Cu") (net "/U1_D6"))
 (segment (start 104.727208 128.312792) (end 149.147208 128.312792) (width 0.2) (layer "B.Cu") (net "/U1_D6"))
 (segment (start 101 129.5) (end 102.587208 127.912792) (width 0.2) (layer "B.Cu") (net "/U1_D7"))
 (segment (start 102.587208 127.912792) (end 147.007208 127.912792) (width 0.2) (layer "B.Cu") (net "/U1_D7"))
 (segment (start 147.007208 127.912792) (end 164.345 110.575) (width 0.2) (layer "B.Cu") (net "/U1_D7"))
 (segment (start 101 126.96) (end 143.9 126.96) (width 0.2) (layer "B.Cu") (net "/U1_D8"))
 (segment (start 143.9 126.96) (end 160.285 110.575) (width 0.2) (layer "B.Cu") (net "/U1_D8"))
 (segment (start 101 124.42) (end 143.9 124.42) (width 0.2) (layer "B.Cu") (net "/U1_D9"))
 (segment (start 143.9 124.42) (end 157.745 110.575) (width 0.2) (layer "B.Cu") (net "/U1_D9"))
 (segment (start 153.765 111.030635) (end 153.120635 111.675) (width 0.2) (layer "F.Cu") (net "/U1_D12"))
 (segment (start 153.765 110.040686) (end 153.765 111.030635) (width 0.2) (layer "F.Cu") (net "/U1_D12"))
 (segment (start 151.225 111.675) (end 150.125 110.575) (width 0.2) (layer "F.Cu") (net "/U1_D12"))
 (segment (start 230.5 85) (end 178.805686 85) (width 0.2) (layer "F.Cu") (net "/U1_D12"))
 (segment (start 153.120635 111.675) (end 151.225 111.675) (width 0.2) (layer "F.Cu") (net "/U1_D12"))
 (segment (start 178.805686 85) (end 153.765 110.040686) (width 0.2) (layer "F.Cu") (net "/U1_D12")))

